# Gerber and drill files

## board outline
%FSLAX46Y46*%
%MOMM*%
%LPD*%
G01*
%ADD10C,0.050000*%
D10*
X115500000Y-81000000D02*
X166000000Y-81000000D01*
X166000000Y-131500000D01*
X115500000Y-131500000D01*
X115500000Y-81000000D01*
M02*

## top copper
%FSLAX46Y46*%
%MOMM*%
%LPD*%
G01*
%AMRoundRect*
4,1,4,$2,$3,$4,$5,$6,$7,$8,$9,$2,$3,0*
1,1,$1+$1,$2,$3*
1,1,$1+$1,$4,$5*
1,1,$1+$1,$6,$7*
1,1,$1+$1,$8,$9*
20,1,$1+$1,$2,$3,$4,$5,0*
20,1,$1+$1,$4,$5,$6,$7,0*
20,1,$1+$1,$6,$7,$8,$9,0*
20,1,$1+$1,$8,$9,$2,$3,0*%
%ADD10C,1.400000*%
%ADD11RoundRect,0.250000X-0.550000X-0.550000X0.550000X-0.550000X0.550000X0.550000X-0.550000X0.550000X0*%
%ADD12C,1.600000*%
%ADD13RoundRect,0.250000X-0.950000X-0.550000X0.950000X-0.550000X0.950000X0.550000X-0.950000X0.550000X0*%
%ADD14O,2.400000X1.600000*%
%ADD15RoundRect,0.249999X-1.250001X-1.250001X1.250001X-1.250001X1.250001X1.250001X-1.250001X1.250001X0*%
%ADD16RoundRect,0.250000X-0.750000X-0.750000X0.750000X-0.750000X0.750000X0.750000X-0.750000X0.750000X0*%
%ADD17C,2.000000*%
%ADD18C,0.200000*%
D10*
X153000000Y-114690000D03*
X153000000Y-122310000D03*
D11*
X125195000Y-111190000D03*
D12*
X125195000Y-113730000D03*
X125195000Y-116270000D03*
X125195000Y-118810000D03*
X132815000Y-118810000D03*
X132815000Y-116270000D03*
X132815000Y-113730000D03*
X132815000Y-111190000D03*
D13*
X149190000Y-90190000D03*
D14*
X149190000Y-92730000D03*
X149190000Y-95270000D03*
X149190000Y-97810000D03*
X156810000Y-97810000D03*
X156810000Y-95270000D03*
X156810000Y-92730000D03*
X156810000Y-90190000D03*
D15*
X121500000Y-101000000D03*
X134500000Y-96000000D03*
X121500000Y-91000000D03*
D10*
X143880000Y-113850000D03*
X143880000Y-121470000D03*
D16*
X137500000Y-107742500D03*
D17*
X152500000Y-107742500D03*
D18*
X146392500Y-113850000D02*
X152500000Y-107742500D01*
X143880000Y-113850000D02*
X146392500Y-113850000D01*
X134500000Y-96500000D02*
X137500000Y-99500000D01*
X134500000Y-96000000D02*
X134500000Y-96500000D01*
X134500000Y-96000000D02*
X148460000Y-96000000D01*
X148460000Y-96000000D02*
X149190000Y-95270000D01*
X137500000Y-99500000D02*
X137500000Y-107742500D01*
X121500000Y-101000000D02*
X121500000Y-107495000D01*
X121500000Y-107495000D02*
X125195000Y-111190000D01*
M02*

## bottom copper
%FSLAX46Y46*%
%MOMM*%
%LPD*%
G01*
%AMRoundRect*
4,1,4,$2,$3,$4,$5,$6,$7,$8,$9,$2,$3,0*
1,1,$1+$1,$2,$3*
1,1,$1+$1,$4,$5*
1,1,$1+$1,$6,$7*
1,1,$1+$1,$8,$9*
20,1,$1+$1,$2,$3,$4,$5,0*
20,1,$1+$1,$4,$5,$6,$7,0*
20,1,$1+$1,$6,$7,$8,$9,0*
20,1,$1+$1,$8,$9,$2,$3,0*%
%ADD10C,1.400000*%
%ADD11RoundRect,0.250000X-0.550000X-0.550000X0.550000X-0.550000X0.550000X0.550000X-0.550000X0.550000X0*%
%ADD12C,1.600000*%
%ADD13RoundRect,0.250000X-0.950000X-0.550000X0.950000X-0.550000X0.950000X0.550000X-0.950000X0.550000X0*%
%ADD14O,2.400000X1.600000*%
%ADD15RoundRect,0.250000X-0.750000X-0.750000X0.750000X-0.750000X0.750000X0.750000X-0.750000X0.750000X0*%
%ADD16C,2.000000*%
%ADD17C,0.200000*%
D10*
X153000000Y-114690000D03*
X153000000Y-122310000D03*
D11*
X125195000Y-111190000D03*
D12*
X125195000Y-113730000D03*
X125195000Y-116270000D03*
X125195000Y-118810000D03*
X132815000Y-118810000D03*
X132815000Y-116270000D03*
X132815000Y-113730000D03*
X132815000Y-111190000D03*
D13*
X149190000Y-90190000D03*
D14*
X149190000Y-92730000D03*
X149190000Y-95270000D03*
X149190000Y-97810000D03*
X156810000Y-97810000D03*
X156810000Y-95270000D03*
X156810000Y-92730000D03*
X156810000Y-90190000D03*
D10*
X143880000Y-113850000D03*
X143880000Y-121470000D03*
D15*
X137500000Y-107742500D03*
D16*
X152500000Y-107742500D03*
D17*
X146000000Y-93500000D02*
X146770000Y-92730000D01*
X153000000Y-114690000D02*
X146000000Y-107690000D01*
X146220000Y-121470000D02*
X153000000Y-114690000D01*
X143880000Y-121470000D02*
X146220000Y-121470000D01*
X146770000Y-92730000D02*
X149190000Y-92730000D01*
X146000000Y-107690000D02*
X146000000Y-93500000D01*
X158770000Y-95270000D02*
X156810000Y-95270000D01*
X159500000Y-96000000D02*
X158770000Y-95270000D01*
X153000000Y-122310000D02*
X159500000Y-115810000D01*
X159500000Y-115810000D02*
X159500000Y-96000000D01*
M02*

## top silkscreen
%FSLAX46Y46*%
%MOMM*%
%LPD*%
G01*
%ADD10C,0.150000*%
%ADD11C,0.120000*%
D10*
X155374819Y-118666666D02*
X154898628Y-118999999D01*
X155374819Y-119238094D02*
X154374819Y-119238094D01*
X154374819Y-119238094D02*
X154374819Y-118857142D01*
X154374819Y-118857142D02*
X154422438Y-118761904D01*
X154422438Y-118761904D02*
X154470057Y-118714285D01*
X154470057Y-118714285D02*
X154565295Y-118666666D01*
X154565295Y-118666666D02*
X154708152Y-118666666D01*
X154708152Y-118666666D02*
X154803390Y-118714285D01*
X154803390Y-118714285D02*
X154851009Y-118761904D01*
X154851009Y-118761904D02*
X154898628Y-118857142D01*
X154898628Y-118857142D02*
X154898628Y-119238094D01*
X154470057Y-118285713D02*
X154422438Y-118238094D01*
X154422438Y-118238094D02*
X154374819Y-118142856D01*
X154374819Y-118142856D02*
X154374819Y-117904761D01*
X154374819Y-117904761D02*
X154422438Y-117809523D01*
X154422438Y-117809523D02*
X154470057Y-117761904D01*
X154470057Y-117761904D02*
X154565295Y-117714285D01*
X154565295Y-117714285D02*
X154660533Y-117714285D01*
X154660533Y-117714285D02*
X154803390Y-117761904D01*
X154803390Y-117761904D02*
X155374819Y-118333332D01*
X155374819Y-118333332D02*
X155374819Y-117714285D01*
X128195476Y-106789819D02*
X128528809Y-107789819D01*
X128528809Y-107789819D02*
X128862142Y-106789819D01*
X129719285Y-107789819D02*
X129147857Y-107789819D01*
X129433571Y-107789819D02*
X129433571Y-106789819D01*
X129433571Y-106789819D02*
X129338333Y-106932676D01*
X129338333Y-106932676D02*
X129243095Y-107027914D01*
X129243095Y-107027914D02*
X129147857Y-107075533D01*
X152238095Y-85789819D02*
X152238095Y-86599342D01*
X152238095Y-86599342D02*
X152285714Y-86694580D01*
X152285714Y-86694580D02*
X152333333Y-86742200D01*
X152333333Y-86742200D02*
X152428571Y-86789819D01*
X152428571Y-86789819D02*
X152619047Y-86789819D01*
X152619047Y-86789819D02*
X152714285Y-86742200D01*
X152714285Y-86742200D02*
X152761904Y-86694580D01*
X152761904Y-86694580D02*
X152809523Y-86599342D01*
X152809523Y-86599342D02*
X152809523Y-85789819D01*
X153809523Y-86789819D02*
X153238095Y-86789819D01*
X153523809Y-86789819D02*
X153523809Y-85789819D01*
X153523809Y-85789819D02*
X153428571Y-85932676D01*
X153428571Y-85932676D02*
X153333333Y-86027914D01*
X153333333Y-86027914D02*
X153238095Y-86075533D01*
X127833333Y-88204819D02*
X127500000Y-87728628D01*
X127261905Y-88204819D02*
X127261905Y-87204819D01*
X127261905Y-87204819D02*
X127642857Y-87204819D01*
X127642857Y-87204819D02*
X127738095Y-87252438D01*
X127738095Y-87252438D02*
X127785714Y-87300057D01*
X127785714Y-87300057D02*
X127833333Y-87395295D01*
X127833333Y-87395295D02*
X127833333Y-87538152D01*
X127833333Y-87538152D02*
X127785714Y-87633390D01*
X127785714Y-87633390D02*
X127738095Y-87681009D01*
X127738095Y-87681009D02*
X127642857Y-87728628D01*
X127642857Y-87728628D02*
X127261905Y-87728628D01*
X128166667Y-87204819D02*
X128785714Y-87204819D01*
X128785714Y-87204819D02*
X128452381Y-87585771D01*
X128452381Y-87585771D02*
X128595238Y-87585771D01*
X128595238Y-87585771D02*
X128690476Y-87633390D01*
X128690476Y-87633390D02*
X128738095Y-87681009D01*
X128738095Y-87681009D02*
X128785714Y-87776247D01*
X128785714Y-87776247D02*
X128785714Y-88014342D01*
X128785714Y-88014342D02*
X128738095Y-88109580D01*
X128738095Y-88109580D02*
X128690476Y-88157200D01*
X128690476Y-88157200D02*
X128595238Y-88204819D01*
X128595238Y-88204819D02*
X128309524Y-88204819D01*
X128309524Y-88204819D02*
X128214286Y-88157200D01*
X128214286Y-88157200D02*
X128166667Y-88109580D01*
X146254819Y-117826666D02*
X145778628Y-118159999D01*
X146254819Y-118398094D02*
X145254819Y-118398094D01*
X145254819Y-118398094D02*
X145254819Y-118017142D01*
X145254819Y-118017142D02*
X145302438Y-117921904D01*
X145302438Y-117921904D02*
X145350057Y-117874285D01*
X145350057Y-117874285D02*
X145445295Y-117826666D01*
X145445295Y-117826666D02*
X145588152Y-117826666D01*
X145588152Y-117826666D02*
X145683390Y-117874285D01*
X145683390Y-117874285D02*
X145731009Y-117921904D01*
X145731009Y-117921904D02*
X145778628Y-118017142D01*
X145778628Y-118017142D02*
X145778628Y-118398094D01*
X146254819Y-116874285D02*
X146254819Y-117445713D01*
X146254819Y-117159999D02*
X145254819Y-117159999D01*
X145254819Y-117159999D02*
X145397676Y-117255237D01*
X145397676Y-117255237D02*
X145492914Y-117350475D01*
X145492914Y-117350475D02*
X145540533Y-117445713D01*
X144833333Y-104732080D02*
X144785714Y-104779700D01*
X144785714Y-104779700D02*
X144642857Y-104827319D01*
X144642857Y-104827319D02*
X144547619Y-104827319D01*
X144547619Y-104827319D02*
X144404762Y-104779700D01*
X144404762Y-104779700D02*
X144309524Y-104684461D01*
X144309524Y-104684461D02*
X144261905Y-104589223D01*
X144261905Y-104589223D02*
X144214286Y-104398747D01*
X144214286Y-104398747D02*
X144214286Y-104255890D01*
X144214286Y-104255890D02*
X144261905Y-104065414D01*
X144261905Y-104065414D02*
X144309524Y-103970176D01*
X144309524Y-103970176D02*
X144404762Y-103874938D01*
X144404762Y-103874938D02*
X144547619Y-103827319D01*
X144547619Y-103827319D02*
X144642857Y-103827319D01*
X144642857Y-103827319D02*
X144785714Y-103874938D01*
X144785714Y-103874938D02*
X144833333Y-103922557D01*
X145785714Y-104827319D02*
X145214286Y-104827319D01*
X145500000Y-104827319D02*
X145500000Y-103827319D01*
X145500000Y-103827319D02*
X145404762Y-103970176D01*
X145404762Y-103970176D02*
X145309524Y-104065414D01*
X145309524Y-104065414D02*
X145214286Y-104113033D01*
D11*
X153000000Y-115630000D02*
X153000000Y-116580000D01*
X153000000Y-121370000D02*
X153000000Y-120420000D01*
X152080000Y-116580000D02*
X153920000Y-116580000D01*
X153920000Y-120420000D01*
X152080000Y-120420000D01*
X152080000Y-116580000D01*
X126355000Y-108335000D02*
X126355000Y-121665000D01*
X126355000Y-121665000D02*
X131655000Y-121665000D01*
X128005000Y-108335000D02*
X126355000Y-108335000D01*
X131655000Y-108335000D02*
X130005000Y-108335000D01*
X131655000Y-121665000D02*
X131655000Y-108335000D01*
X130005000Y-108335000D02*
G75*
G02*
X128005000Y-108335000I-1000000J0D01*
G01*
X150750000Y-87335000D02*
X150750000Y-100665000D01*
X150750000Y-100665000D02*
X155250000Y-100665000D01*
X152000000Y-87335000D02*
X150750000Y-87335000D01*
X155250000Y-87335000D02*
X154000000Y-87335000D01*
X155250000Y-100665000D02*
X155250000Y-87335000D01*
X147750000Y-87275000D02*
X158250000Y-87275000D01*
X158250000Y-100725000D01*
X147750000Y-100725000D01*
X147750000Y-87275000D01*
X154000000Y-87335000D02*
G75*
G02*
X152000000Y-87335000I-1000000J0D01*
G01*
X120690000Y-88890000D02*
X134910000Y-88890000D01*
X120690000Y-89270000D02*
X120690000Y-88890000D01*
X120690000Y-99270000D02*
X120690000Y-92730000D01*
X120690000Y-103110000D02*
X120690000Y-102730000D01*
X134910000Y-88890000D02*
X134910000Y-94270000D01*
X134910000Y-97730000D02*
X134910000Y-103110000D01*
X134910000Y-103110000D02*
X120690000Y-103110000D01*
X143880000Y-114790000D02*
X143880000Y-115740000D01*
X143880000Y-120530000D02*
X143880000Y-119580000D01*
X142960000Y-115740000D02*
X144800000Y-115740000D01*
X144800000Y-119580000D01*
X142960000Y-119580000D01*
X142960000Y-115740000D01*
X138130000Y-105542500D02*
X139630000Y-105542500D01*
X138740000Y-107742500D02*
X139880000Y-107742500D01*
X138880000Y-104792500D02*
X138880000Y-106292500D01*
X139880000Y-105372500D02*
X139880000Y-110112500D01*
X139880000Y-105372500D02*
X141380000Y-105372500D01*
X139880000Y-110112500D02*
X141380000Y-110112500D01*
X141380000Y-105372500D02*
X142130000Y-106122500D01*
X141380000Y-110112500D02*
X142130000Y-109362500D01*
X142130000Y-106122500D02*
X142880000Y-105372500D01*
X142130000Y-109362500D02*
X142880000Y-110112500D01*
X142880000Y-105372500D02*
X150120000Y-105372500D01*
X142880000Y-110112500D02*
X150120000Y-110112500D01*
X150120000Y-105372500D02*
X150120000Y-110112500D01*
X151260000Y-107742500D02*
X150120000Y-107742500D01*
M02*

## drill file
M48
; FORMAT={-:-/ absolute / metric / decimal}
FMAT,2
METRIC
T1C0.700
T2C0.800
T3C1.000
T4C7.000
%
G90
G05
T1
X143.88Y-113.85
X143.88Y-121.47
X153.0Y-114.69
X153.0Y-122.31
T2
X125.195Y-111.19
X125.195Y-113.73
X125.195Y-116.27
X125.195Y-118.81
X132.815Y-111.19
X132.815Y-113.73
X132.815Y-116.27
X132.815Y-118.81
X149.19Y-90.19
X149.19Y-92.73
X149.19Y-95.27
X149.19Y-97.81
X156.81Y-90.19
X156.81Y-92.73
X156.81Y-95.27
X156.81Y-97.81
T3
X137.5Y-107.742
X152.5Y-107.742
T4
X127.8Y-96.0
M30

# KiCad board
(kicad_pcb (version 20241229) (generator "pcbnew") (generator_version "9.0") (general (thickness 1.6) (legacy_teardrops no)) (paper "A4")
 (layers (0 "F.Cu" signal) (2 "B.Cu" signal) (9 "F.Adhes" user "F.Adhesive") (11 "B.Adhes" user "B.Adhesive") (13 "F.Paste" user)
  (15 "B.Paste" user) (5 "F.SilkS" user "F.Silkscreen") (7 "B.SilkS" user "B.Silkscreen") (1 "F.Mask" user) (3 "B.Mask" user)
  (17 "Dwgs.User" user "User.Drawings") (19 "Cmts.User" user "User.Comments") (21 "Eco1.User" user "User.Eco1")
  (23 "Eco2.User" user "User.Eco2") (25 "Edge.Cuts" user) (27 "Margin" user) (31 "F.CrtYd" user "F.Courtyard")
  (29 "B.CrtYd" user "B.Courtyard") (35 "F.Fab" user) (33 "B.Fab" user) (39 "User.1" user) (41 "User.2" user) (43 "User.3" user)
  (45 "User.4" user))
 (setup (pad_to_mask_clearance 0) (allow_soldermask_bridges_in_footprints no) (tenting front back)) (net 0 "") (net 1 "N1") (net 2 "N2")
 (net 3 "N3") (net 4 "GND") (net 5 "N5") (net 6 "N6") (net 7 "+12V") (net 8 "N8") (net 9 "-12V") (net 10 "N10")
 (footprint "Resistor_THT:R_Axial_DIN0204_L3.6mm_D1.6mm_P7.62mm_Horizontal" (layer "F.Cu") (at 153 114.69 -90)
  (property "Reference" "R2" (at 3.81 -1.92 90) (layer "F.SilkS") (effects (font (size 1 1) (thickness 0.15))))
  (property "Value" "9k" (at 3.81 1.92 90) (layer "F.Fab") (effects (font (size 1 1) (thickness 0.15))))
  (fp_line (start 0.94 0) (end 1.89 0) (stroke (width 0.12) (type solid)) (layer "F.SilkS"))
  (fp_line (start 6.68 0) (end 5.73 0) (stroke (width 0.12) (type solid)) (layer "F.SilkS"))
  (fp_rect (start 1.89 -0.92) (end 5.73 0.92) (stroke (width 0.12) (type solid)) (fill no) (layer "F.SilkS"))
  (pad "1" thru_hole circle (at 0 0 270) (size 1.4 1.4) (drill 0.7) (layers "*.Cu" "*.Mask") (remove_unused_layers no) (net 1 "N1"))
  (pad "2" thru_hole circle (at 7.62 0 270) (size 1.4 1.4) (drill 0.7) (layers "*.Cu" "*.Mask") (remove_unused_layers no) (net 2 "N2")))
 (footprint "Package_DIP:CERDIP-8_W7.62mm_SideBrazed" (layer "F.Cu") (at 125.195 111.19)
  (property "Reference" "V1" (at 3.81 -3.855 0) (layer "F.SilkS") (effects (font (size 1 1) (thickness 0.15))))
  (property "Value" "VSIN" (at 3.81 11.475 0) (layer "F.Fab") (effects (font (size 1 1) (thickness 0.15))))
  (fp_line (start 1.16 -2.855) (end 1.16 10.475) (stroke (width 0.12) (type solid)) (layer "F.SilkS"))
  (fp_line (start 1.16 10.475) (end 6.46 10.475) (stroke (width 0.12) (type solid)) (layer "F.SilkS"))
  (fp_line (start 2.81 -2.855) (end 1.16 -2.855) (stroke (width 0.12) (type solid)) (layer "F.SilkS"))
  (fp_line (start 6.46 -2.855) (end 4.81 -2.855) (stroke (width 0.12) (type solid)) (layer "F.SilkS"))
  (fp_line (start 6.46 10.475) (end 6.46 -2.855) (stroke (width 0.12) (type solid)) (layer "F.SilkS"))
  (fp_arc (start 4.81 -2.855) (mid 3.81 -1.855) (end 2.81 -2.855) (stroke (width 0.12) (type solid)) (layer "F.SilkS"))
  (pad "1" thru_hole roundrect (at 0 0) (size 1.6 1.6) (drill 0.8) (layers "*.Cu" "*.Mask") (remove_unused_layers no)
   (roundrect_rratio 0.15625) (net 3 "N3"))
  (pad "2" thru_hole circle (at 0 2.54) (size 1.6 1.6) (drill 0.8) (layers "*.Cu" "*.Mask") (remove_unused_layers no) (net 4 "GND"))
  (pad "3" thru_hole circle (at 0 5.08) (size 1.6 1.6) (drill 0.8) (layers "*.Cu" "*.Mask") (remove_unused_layers no))
  (pad "4" thru_hole circle (at 0 7.62) (size 1.6 1.6) (drill 0.8) (layers "*.Cu" "*.Mask") (remove_unused_layers no))
  (pad "5" thru_hole circle (at 7.62 7.62) (size 1.6 1.6) (drill 0.8) (layers "*.Cu" "*.Mask") (remove_unused_layers no))
  (pad "6" thru_hole circle (at 7.62 5.08) (size 1.6 1.6) (drill 0.8) (layers "*.Cu" "*.Mask") (remove_unused_layers no))
  (pad "7" thru_hole circle (at 7.62 2.54) (size 1.6 1.6) (drill 0.8) (layers "*.Cu" "*.Mask") (remove_unused_layers no))
  (pad "8" thru_hole circle (at 7.62 0) (size 1.6 1.6) (drill 0.8) (layers "*.Cu" "*.Mask") (remove_unused_layers no)))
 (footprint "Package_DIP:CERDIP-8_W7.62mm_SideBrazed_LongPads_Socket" (layer "F.Cu") (at 149.19 90.19)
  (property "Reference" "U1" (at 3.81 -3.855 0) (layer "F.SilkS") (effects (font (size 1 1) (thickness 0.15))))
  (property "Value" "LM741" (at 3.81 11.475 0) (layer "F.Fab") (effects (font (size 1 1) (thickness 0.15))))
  (fp_line (start 1.56 -2.855) (end 1.56 10.475) (stroke (width 0.12) (type solid)) (layer "F.SilkS"))
  (fp_line (start 1.56 10.475) (end 6.06 10.475) (stroke (width 0.12) (type solid)) (layer "F.SilkS"))
  (fp_line (start 2.81 -2.855) (end 1.56 -2.855) (stroke (width 0.12) (type solid)) (layer "F.SilkS"))
  (fp_line (start 6.06 -2.855) (end 4.81 -2.855) (stroke (width 0.12) (type solid)) (layer "F.SilkS"))
  (fp_line (start 6.06 10.475) (end 6.06 -2.855) (stroke (width 0.12) (type solid)) (layer "F.SilkS"))
  (fp_rect (start -1.44 -2.915) (end 9.06 10.535) (stroke (width 0.12) (type solid)) (fill no) (layer "F.SilkS"))
  (fp_arc (start 4.81 -2.855) (mid 3.81 -1.855) (end 2.81 -2.855) (stroke (width 0.12) (type solid)) (layer "F.SilkS"))
  (pad "1" thru_hole roundrect (at 0 0) (size 2.4 1.6) (drill 0.8) (layers "*.Cu" "*.Mask") (remove_unused_layers no)
   (roundrect_rratio 0.15625) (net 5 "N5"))
  (pad "2" thru_hole oval (at 0 2.54) (size 2.4 1.6) (drill 0.8) (layers "*.Cu" "*.Mask") (remove_unused_layers no) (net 1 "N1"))
  (pad "3" thru_hole oval (at 0 5.08) (size 2.4 1.6) (drill 0.8) (layers "*.Cu" "*.Mask") (remove_unused_layers no) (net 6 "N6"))
  (pad "4" thru_hole oval (at 0 7.62) (size 2.4 1.6) (drill 0.8) (layers "*.Cu" "*.Mask") (remove_unused_layers no) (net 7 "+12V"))
  (pad "5" thru_hole oval (at 7.62 7.62) (size 2.4 1.6) (drill 0.8) (layers "*.Cu" "*.Mask") (remove_unused_layers no) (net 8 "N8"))
  (pad "6" thru_hole oval (at 7.62 5.08) (size 2.4 1.6) (drill 0.8) (layers "*.Cu" "*.Mask") (remove_unused_layers no) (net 2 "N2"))
  (pad "7" thru_hole oval (at 7.62 2.54) (size 2.4 1.6) (drill 0.8) (layers "*.Cu" "*.Mask") (remove_unused_layers no) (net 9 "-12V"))
  (pad "8" thru_hole oval (at 7.62 0) (size 2.4 1.6) (drill 0.8) (layers "*.Cu" "*.Mask") (remove_unused_layers no) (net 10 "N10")))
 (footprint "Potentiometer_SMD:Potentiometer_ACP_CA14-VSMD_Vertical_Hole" (layer "F.Cu") (at 128 96)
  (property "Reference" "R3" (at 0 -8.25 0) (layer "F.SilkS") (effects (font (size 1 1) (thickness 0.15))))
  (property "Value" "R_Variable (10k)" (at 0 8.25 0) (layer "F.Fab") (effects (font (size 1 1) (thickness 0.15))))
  (fp_line (start -7.31 -7.11) (end 6.91 -7.11) (stroke (width 0.12) (type solid)) (layer "F.SilkS"))
  (fp_line (start -7.31 -6.73) (end -7.31 -7.11) (stroke (width 0.12) (type solid)) (layer "F.SilkS"))
  (fp_line (start -7.31 3.27) (end -7.31 -3.27) (stroke (width 0.12) (type solid)) (layer "F.SilkS"))
  (fp_line (start -7.31 7.11) (end -7.31 6.73) (stroke (width 0.12) (type solid)) (layer "F.SilkS"))
  (fp_line (start 6.91 -7.11) (end 6.91 -1.73) (stroke (width 0.12) (type solid)) (layer "F.SilkS"))
  (fp_line (start 6.91 1.73) (end 6.91 7.11) (stroke (width 0.12) (type solid)) (layer "F.SilkS"))
  (fp_line (start 6.91 7.11) (end -7.31 7.11) (stroke (width 0.12) (type solid)) (layer "F.SilkS"))
  (pad "" np_thru_hole circle (at -0.2 0) (size 7 7) (drill 7) (layers "*.Cu" "*.Mask"))
  (pad "1" smd roundrect (at -6.5 5) (size 3 3) (layers "F.Cu" "F.Mask" "F.Paste") (roundrect_rratio 0.083333) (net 3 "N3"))
  (pad "2" smd roundrect (at 6.5 0) (size 3 3) (layers "F.Cu" "F.Mask" "F.Paste") (roundrect_rratio 0.083333) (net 6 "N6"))
  (pad "3" smd roundrect (at -6.5 -5) (size 3 3) (layers "F.Cu" "F.Mask" "F.Paste") (roundrect_rratio 0.083333)))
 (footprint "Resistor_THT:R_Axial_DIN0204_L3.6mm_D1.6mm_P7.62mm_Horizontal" (layer "F.Cu") (at 143.88 113.85 -90)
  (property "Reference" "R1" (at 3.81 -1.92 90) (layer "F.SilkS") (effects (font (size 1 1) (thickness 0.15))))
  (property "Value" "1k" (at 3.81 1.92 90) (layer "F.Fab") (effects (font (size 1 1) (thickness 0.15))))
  (fp_line (start 0.94 0) (end 1.89 0) (stroke (width 0.12) (type solid)) (layer "F.SilkS"))
  (fp_line (start 6.68 0) (end 5.73 0) (stroke (width 0.12) (type solid)) (layer "F.SilkS"))
  (fp_rect (start 1.89 -0.92) (end 5.73 0.92) (stroke (width 0.12) (type solid)) (fill no) (layer "F.SilkS"))
  (pad "1" thru_hole circle (at 0 0 270) (size 1.4 1.4) (drill 0.7) (layers "*.Cu" "*.Mask") (remove_unused_layers no) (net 4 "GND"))
  (pad "2" thru_hole circle (at 7.62 0 270) (size 1.4 1.4) (drill 0.7) (layers "*.Cu" "*.Mask") (remove_unused_layers no) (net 1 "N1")))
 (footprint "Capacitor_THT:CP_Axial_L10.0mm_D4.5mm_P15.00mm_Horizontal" (layer "F.Cu") (at 137.5 107.7425)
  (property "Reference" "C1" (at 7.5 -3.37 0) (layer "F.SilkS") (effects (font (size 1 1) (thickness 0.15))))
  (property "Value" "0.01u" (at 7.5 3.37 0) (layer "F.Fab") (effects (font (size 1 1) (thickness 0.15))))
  (fp_line (start 0.63 -2.2) (end 2.13 -2.2) (stroke (width 0.12) (type solid)) (layer "F.SilkS"))
  (fp_line (start 1.24 0) (end 2.38 0) (stroke (width 0.12) (type solid)) (layer "F.SilkS"))
  (fp_line (start 1.38 -2.95) (end 1.38 -1.45) (stroke (width 0.12) (type solid)) (layer "F.SilkS"))
  (fp_line (start 2.38 -2.37) (end 2.38 2.37) (stroke (width 0.12) (type solid)) (layer "F.SilkS"))
  (fp_line (start 2.38 -2.37) (end 3.88 -2.37) (stroke (width 0.12) (type solid)) (layer "F.SilkS"))
  (fp_line (start 2.38 2.37) (end 3.88 2.37) (stroke (width 0.12) (type solid)) (layer "F.SilkS"))
  (fp_line (start 3.88 -2.37) (end 4.63 -1.62) (stroke (width 0.12) (type solid)) (layer "F.SilkS"))
  (fp_line (start 3.88 2.37) (end 4.63 1.62) (stroke (width 0.12) (type solid)) (layer "F.SilkS"))
  (fp_line (start 4.63 -1.62) (end 5.38 -2.37) (stroke (width 0.12) (type solid)) (layer "F.SilkS"))
  (fp_line (start 4.63 1.62) (end 5.38 2.37) (stroke (width 0.12) (type solid)) (layer "F.SilkS"))
  (fp_line (start 5.38 -2.37) (end 12.62 -2.37) (stroke (width 0.12) (type solid)) (layer "F.SilkS"))
  (fp_line (start 5.38 2.37) (end 12.62 2.37) (stroke (width 0.12) (type solid)) (layer "F.SilkS"))
  (fp_line (start 12.62 -2.37) (end 12.62 2.37) (stroke (width 0.12) (type solid)) (layer "F.SilkS"))
  (fp_line (start 13.76 0) (end 12.62 0) (stroke (width 0.12) (type solid)) (layer "F.SilkS"))
  (pad "1" thru_hole roundrect (at 0 0) (size 2 2) (drill 1) (layers "*.Cu" "*.Mask") (remove_unused_layers no) (roundrect_rratio 0.125)
   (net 6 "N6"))
  (pad "2" thru_hole circle (at 15 0) (size 2 2) (drill 1) (layers "*.Cu" "*.Mask") (remove_unused_layers no) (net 4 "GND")))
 (gr_rect (start 115.5 81) (end 166 131.5) (stroke (width 0.05) (type default)) (fill no) (layer "Edge.Cuts"))
 (segment (start 146.3925 113.85) (end 152.5 107.7425) (width 0.2) (layer "F.Cu") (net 4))
 (segment (start 143.88 113.85) (end 146.3925 113.85) (width 0.2) (layer "F.Cu") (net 4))
 (segment (start 134.5 96.5) (end 137.5 99.5) (width 0.2) (layer "F.Cu") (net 6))
 (segment (start 134.5 96) (end 134.5 96.5) (width 0.2) (layer "F.Cu") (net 6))
 (segment (start 134.5 96) (end 148.46 96) (width 0.2) (layer "F.Cu") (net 6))
 (segment (start 148.46 96) (end 149.19 95.27) (width 0.2) (layer "F.Cu") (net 6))
 (segment (start 137.5 99.5) (end 137.5 107.7425) (width 0.2) (layer "F.Cu") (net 6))
 (segment (start 146 93.5) (end 146.77 92.73) (width 0.2) (layer "B.Cu") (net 1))
 (segment (start 153 114.69) (end 146 107.69) (width 0.2) (layer "B.Cu") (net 1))
 (segment (start 146.22 121.47) (end 153 114.69) (width 0.2) (layer "B.Cu") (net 1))
 (segment (start 143.88 121.47) (end 146.22 121.47) (width 0.2) (layer "B.Cu") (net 1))
 (segment (start 146.77 92.73) (end 149.19 92.73) (width 0.2) (layer "B.Cu") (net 1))
 (segment (start 146 107.69) (end 146 93.5) (width 0.2) (layer "B.Cu") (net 1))
 (segment (start 158.77 95.27) (end 156.81 95.27) (width 0.2) (layer "B.Cu") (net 2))
 (segment (start 159.5 96) (end 158.77 95.27) (width 0.2) (layer "B.Cu") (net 2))
 (segment (start 153 122.31) (end 159.5 115.81) (width 0.2) (layer "B.Cu") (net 2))
 (segment (start 159.5 115.81) (end 159.5 96) (width 0.2) (layer "B.Cu") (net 2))
 (segment (start 121.5 101) (end 121.5 107.495) (width 0.2) (layer "F.Cu") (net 3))
 (segment (start 121.5 107.495) (end 125.195 111.19) (width 0.2) (layer "F.Cu") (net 3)))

